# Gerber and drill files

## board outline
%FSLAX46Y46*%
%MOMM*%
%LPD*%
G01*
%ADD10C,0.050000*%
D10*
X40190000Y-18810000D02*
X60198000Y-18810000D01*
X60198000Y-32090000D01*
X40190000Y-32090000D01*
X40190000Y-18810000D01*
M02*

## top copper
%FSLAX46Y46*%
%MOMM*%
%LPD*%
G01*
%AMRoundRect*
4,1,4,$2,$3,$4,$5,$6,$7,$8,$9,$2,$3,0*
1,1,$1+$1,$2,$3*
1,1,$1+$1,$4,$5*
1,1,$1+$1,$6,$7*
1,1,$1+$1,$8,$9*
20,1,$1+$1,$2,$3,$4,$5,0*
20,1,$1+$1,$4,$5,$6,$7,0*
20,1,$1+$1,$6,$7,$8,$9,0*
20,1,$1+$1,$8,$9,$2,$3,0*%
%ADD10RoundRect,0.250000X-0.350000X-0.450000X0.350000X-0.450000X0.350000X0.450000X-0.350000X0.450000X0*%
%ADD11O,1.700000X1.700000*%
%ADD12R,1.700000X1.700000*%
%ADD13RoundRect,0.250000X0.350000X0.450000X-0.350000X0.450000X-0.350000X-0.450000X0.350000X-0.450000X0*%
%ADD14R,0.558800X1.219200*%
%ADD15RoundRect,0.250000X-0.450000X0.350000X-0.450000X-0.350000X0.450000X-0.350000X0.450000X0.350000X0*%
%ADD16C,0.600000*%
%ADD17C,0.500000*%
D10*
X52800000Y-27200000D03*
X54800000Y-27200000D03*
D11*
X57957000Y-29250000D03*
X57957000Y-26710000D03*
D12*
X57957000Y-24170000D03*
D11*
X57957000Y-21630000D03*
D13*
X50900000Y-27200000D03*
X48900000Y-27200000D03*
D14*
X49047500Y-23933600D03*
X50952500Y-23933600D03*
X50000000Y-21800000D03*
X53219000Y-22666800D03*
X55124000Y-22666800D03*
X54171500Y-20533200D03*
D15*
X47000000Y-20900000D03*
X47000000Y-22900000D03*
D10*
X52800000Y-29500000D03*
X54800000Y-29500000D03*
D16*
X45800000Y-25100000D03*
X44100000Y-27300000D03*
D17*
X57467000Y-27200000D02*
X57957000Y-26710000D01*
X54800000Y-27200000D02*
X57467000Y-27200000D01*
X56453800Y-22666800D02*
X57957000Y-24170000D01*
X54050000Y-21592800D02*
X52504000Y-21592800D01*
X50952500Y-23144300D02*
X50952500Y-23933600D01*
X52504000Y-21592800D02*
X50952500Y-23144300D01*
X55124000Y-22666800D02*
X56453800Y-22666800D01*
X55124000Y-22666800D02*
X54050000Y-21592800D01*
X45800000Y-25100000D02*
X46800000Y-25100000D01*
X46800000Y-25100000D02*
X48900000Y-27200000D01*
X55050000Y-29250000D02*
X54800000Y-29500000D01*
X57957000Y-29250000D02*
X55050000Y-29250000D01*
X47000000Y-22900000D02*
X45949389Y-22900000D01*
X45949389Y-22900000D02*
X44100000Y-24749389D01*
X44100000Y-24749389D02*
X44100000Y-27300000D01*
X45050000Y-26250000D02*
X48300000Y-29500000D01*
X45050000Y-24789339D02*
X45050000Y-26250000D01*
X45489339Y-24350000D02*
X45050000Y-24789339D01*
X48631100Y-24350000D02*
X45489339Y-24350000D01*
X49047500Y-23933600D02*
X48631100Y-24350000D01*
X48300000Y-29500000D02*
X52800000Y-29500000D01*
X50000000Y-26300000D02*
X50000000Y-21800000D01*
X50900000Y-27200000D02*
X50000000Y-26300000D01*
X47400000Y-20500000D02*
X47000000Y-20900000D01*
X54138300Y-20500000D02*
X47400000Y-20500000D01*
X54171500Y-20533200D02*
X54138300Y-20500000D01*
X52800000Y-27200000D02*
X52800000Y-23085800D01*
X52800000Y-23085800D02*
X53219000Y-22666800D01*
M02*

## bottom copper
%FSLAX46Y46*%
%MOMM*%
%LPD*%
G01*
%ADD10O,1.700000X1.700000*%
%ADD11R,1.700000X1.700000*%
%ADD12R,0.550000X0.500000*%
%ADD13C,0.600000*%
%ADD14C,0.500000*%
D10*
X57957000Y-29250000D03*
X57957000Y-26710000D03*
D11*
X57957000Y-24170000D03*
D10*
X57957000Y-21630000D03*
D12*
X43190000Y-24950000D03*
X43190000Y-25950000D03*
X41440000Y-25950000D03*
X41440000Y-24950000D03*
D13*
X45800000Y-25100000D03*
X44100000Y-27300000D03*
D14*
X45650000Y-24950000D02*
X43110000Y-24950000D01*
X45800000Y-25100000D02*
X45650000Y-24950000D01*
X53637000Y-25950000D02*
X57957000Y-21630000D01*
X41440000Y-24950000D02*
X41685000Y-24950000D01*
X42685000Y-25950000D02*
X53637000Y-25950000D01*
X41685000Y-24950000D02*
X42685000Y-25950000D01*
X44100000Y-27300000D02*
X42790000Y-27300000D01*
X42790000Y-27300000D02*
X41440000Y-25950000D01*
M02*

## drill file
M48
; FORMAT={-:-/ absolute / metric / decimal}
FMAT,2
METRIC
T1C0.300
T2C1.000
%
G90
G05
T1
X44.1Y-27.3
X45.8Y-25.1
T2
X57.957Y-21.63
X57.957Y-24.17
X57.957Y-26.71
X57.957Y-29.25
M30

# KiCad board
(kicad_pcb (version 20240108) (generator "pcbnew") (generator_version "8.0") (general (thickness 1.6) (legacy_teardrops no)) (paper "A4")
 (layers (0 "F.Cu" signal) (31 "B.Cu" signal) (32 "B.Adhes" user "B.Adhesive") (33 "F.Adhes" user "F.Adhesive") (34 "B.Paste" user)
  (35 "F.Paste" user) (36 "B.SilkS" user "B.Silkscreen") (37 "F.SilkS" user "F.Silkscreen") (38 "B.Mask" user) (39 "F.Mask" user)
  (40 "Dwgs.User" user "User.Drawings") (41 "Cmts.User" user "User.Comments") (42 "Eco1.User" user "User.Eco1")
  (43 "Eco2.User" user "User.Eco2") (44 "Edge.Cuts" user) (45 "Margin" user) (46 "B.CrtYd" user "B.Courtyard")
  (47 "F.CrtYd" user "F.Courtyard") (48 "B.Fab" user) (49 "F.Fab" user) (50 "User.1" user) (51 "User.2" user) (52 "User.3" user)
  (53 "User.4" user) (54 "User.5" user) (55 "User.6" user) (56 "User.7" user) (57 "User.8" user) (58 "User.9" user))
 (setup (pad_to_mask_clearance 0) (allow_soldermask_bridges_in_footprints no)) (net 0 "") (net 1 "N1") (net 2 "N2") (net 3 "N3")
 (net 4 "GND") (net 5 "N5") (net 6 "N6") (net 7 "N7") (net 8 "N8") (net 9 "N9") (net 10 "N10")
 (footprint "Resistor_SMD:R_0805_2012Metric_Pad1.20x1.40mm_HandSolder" (layer "F.Cu") (at 53.8 27.2)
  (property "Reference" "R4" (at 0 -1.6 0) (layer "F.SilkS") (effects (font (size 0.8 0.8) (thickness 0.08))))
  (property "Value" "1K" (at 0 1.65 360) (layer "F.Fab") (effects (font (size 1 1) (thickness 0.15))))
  (pad "1" smd roundrect (at -1 0) (size 1.2 1.4) (layers "F.Cu" "F.Paste" "F.Mask") (roundrect_rratio 0.208333) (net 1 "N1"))
  (pad "2" smd roundrect (at 1 0) (size 1.2 1.4) (layers "F.Cu" "F.Paste" "F.Mask") (roundrect_rratio 0.208333) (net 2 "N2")))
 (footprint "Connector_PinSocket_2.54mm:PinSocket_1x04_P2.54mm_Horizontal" (layer "F.Cu") (at 57.957 29.25 180)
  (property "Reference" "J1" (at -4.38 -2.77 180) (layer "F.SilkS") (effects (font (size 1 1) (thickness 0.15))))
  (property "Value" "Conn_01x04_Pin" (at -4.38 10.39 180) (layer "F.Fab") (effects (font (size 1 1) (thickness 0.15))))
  (pad "1" thru_hole oval (at 0 0 180) (size 1.7 1.7) (drill 1) (layers "*.Cu" "*.Mask") (remove_unused_layers no) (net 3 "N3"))
  (pad "2" thru_hole oval (at 0 2.54 180) (size 1.7 1.7) (drill 1) (layers "*.Cu" "*.Mask") (remove_unused_layers no) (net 2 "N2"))
  (pad "3" thru_hole rect (at 0 5.08 180) (size 1.7 1.7) (drill 1) (layers "*.Cu" "*.Mask") (remove_unused_layers no) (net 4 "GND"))
  (pad "4" thru_hole oval (at 0 7.62 180) (size 1.7 1.7) (drill 1) (layers "*.Cu" "*.Mask") (remove_unused_layers no) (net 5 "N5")))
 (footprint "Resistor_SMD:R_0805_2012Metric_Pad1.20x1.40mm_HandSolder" (layer "F.Cu") (at 49.9 27.2 180)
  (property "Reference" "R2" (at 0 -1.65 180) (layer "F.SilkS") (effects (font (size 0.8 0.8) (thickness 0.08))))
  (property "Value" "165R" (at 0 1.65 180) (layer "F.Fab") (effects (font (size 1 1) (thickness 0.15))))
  (pad "1" smd roundrect (at -1 0 180) (size 1.2 1.4) (layers "F.Cu" "F.Paste" "F.Mask") (roundrect_rratio 0.208333) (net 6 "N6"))
  (pad "2" smd roundrect (at 1 0 180) (size 1.2 1.4) (layers "F.Cu" "F.Paste" "F.Mask") (roundrect_rratio 0.208333) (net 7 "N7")))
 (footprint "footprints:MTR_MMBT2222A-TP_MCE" (layer "F.Cu") (at 50 22.8668)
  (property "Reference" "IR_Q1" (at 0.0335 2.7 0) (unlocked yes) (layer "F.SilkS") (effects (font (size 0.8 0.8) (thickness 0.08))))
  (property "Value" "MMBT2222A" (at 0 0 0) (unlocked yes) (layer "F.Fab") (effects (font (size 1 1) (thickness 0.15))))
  (pad "1" smd rect (at -0.9525 1.0668) (size 0.5588 1.2192) (layers "F.Cu" "F.Paste" "F.Mask") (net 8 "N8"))
  (pad "2" smd rect (at 0.9525 1.0668) (size 0.5588 1.2192) (layers "F.Cu" "F.Paste" "F.Mask") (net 4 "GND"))
  (pad "3" smd rect (at 0 -1.0668) (size 0.5588 1.2192) (layers "F.Cu" "F.Paste" "F.Mask") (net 6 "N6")))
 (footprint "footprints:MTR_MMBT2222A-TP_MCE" (layer "F.Cu") (at 54.1715 21.6)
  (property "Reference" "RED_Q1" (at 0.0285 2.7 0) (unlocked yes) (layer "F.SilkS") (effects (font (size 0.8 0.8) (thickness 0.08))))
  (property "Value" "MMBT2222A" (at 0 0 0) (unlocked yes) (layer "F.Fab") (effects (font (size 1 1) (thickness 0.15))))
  (pad "1" smd rect (at -0.9525 1.0668) (size 0.5588 1.2192) (layers "F.Cu" "F.Paste" "F.Mask") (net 1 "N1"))
  (pad "2" smd rect (at 0.9525 1.0668) (size 0.5588 1.2192) (layers "F.Cu" "F.Paste" "F.Mask") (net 4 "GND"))
  (pad "3" smd rect (at 0 -1.0668) (size 0.5588 1.2192) (layers "F.Cu" "F.Paste" "F.Mask") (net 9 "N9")))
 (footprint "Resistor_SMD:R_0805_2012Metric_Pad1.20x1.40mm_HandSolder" (layer "F.Cu") (at 47 21.9 -90)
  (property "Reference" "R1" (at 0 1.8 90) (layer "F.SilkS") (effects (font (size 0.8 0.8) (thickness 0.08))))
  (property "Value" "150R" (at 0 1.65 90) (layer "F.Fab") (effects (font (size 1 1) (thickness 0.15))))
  (pad "1" smd roundrect (at -1 0 270) (size 1.2 1.4) (layers "F.Cu" "F.Paste" "F.Mask") (roundrect_rratio 0.208333) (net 9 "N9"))
  (pad "2" smd roundrect (at 1 0 270) (size 1.2 1.4) (layers "F.Cu" "F.Paste" "F.Mask") (roundrect_rratio 0.208333) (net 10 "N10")))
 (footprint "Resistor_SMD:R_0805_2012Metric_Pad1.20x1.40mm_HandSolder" (layer "F.Cu") (at 53.8 29.5)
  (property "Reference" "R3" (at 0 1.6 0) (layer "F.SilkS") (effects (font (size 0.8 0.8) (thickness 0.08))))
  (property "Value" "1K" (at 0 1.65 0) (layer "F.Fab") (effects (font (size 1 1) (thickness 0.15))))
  (pad "1" smd roundrect (at -1 0) (size 1.2 1.4) (layers "F.Cu" "F.Paste" "F.Mask") (roundrect_rratio 0.208333) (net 8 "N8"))
  (pad "2" smd roundrect (at 1 0) (size 1.2 1.4) (layers "F.Cu" "F.Paste" "F.Mask") (roundrect_rratio 0.208333) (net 3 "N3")))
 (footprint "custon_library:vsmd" (layer "B.Cu") (at 43.28 25.01 180)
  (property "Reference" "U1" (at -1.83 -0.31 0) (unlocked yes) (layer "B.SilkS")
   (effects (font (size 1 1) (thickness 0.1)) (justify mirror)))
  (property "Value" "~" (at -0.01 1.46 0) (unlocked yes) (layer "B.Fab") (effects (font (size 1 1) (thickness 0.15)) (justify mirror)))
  (pad "1" smd rect (at 0.09 0.06 180) (size 0.55 0.5) (layers "B.Cu" "B.Paste" "B.Mask") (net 7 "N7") (solder_mask_margin 0.05)
   (thermal_bridge_angle 45))
  (pad "2" smd rect (at 0.09 -0.94 180) (size 0.55 0.5) (layers "B.Cu" "B.Paste" "B.Mask") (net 5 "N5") (solder_mask_margin 0.05)
   (thermal_bridge_angle 45))
  (pad "3" smd rect (at 1.84 -0.94 180) (size 0.55 0.5) (layers "B.Cu" "B.Paste" "B.Mask") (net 10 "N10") (solder_mask_margin 0.05)
   (thermal_bridge_angle 45))
  (pad "4" smd rect (at 1.84 0.06 180) (size 0.55 0.5) (layers "B.Cu" "B.Paste" "B.Mask") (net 5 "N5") (solder_mask_margin 0.05)
   (thermal_bridge_angle 45)))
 (gr_rect (start 40.19 18.81) (end 60.198 32.09) (stroke (width 0.05) (type default)) (fill none) (layer "Edge.Cuts"))
 (segment (start 57.467 27.2) (end 57.957 26.71) (width 0.5) (layer "F.Cu") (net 2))
 (segment (start 54.8 27.2) (end 57.467 27.2) (width 0.5) (layer "F.Cu") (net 2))
 (segment (start 56.4538 22.6668) (end 57.957 24.17) (width 0.5) (layer "F.Cu") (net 4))
 (segment (start 54.05 21.5928) (end 52.504 21.5928) (width 0.5) (layer "F.Cu") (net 4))
 (segment (start 50.9525 23.1443) (end 50.9525 23.9336) (width 0.5) (layer "F.Cu") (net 4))
 (segment (start 52.504 21.5928) (end 50.9525 23.1443) (width 0.5) (layer "F.Cu") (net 4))
 (segment (start 55.124 22.6668) (end 56.4538 22.6668) (width 0.5) (layer "F.Cu") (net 4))
 (segment (start 55.124 22.6668) (end 54.05 21.5928) (width 0.5) (layer "F.Cu") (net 4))
 (segment (start 45.8 25.1) (end 46.8 25.1) (width 0.5) (layer "F.Cu") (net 7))
 (segment (start 46.8 25.1) (end 48.9 27.2) (width 0.5) (layer "F.Cu") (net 7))
 (via (at 45.8 25.1) (size 0.6) (drill 0.3) (layers "F.Cu" "B.Cu") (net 7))
 (segment (start 45.65 24.95) (end 43.11 24.95) (width 0.5) (layer "B.Cu") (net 7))
 (segment (start 45.8 25.1) (end 45.65 24.95) (width 0.5) (layer "B.Cu") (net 7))
 (segment (start 53.637 25.95) (end 57.957 21.63) (width 0.5) (layer "B.Cu") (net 5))
 (segment (start 41.44 24.95) (end 41.685 24.95) (width 0.5) (layer "B.Cu") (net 5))
 (segment (start 42.685 25.95) (end 53.637 25.95) (width 0.5) (layer "B.Cu") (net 5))
 (segment (start 41.685 24.95) (end 42.685 25.95) (width 0.5) (layer "B.Cu") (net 5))
 (segment (start 55.05 29.25) (end 54.8 29.5) (width 0.5) (layer "F.Cu") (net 3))
 (segment (start 57.957 29.25) (end 55.05 29.25) (width 0.5) (layer "F.Cu") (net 3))
 (segment (start 47 22.9) (end 45.949389 22.9) (width 0.5) (layer "F.Cu") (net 10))
 (segment (start 45.949389 22.9) (end 44.1 24.749389) (width 0.5) (layer "F.Cu") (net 10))
 (segment (start 44.1 24.749389) (end 44.1 27.3) (width 0.5) (layer "F.Cu") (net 10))
 (via (at 44.1 27.3) (size 0.6) (drill 0.3) (layers "F.Cu" "B.Cu") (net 10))
 (segment (start 44.1 27.3) (end 42.79 27.3) (width 0.5) (layer "B.Cu") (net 10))
 (segment (start 42.79 27.3) (end 41.44 25.95) (width 0.5) (layer "B.Cu") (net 10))
 (segment (start 45.05 26.25) (end 48.3 29.5) (width 0.5) (layer "F.Cu") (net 8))
 (segment (start 45.05 24.789339) (end 45.05 26.25) (width 0.5) (layer "F.Cu") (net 8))
 (segment (start 45.489339 24.35) (end 45.05 24.789339) (width 0.5) (layer "F.Cu") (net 8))
 (segment (start 48.6311 24.35) (end 45.489339 24.35) (width 0.5) (layer "F.Cu") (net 8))
 (segment (start 49.0475 23.9336) (end 48.6311 24.35) (width 0.5) (layer "F.Cu") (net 8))
 (segment (start 48.3 29.5) (end 52.8 29.5) (width 0.5) (layer "F.Cu") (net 8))
 (segment (start 50 26.3) (end 50 21.8) (width 0.5) (layer "F.Cu") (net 6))
 (segment (start 50.9 27.2) (end 50 26.3) (width 0.5) (layer "F.Cu") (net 6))
 (segment (start 47.4 20.5) (end 47 20.9) (width 0.5) (layer "F.Cu") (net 9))
 (segment (start 54.1383 20.5) (end 47.4 20.5) (width 0.5) (layer "F.Cu") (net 9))
 (segment (start 54.1715 20.5332) (end 54.1383 20.5) (width 0.5) (layer "F.Cu") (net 9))
 (segment (start 52.8 27.2) (end 52.8 23.0858) (width 0.5) (layer "F.Cu") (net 1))
 (segment (start 52.8 23.0858) (end 53.219 22.6668) (width 0.5) (layer "F.Cu") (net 1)))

